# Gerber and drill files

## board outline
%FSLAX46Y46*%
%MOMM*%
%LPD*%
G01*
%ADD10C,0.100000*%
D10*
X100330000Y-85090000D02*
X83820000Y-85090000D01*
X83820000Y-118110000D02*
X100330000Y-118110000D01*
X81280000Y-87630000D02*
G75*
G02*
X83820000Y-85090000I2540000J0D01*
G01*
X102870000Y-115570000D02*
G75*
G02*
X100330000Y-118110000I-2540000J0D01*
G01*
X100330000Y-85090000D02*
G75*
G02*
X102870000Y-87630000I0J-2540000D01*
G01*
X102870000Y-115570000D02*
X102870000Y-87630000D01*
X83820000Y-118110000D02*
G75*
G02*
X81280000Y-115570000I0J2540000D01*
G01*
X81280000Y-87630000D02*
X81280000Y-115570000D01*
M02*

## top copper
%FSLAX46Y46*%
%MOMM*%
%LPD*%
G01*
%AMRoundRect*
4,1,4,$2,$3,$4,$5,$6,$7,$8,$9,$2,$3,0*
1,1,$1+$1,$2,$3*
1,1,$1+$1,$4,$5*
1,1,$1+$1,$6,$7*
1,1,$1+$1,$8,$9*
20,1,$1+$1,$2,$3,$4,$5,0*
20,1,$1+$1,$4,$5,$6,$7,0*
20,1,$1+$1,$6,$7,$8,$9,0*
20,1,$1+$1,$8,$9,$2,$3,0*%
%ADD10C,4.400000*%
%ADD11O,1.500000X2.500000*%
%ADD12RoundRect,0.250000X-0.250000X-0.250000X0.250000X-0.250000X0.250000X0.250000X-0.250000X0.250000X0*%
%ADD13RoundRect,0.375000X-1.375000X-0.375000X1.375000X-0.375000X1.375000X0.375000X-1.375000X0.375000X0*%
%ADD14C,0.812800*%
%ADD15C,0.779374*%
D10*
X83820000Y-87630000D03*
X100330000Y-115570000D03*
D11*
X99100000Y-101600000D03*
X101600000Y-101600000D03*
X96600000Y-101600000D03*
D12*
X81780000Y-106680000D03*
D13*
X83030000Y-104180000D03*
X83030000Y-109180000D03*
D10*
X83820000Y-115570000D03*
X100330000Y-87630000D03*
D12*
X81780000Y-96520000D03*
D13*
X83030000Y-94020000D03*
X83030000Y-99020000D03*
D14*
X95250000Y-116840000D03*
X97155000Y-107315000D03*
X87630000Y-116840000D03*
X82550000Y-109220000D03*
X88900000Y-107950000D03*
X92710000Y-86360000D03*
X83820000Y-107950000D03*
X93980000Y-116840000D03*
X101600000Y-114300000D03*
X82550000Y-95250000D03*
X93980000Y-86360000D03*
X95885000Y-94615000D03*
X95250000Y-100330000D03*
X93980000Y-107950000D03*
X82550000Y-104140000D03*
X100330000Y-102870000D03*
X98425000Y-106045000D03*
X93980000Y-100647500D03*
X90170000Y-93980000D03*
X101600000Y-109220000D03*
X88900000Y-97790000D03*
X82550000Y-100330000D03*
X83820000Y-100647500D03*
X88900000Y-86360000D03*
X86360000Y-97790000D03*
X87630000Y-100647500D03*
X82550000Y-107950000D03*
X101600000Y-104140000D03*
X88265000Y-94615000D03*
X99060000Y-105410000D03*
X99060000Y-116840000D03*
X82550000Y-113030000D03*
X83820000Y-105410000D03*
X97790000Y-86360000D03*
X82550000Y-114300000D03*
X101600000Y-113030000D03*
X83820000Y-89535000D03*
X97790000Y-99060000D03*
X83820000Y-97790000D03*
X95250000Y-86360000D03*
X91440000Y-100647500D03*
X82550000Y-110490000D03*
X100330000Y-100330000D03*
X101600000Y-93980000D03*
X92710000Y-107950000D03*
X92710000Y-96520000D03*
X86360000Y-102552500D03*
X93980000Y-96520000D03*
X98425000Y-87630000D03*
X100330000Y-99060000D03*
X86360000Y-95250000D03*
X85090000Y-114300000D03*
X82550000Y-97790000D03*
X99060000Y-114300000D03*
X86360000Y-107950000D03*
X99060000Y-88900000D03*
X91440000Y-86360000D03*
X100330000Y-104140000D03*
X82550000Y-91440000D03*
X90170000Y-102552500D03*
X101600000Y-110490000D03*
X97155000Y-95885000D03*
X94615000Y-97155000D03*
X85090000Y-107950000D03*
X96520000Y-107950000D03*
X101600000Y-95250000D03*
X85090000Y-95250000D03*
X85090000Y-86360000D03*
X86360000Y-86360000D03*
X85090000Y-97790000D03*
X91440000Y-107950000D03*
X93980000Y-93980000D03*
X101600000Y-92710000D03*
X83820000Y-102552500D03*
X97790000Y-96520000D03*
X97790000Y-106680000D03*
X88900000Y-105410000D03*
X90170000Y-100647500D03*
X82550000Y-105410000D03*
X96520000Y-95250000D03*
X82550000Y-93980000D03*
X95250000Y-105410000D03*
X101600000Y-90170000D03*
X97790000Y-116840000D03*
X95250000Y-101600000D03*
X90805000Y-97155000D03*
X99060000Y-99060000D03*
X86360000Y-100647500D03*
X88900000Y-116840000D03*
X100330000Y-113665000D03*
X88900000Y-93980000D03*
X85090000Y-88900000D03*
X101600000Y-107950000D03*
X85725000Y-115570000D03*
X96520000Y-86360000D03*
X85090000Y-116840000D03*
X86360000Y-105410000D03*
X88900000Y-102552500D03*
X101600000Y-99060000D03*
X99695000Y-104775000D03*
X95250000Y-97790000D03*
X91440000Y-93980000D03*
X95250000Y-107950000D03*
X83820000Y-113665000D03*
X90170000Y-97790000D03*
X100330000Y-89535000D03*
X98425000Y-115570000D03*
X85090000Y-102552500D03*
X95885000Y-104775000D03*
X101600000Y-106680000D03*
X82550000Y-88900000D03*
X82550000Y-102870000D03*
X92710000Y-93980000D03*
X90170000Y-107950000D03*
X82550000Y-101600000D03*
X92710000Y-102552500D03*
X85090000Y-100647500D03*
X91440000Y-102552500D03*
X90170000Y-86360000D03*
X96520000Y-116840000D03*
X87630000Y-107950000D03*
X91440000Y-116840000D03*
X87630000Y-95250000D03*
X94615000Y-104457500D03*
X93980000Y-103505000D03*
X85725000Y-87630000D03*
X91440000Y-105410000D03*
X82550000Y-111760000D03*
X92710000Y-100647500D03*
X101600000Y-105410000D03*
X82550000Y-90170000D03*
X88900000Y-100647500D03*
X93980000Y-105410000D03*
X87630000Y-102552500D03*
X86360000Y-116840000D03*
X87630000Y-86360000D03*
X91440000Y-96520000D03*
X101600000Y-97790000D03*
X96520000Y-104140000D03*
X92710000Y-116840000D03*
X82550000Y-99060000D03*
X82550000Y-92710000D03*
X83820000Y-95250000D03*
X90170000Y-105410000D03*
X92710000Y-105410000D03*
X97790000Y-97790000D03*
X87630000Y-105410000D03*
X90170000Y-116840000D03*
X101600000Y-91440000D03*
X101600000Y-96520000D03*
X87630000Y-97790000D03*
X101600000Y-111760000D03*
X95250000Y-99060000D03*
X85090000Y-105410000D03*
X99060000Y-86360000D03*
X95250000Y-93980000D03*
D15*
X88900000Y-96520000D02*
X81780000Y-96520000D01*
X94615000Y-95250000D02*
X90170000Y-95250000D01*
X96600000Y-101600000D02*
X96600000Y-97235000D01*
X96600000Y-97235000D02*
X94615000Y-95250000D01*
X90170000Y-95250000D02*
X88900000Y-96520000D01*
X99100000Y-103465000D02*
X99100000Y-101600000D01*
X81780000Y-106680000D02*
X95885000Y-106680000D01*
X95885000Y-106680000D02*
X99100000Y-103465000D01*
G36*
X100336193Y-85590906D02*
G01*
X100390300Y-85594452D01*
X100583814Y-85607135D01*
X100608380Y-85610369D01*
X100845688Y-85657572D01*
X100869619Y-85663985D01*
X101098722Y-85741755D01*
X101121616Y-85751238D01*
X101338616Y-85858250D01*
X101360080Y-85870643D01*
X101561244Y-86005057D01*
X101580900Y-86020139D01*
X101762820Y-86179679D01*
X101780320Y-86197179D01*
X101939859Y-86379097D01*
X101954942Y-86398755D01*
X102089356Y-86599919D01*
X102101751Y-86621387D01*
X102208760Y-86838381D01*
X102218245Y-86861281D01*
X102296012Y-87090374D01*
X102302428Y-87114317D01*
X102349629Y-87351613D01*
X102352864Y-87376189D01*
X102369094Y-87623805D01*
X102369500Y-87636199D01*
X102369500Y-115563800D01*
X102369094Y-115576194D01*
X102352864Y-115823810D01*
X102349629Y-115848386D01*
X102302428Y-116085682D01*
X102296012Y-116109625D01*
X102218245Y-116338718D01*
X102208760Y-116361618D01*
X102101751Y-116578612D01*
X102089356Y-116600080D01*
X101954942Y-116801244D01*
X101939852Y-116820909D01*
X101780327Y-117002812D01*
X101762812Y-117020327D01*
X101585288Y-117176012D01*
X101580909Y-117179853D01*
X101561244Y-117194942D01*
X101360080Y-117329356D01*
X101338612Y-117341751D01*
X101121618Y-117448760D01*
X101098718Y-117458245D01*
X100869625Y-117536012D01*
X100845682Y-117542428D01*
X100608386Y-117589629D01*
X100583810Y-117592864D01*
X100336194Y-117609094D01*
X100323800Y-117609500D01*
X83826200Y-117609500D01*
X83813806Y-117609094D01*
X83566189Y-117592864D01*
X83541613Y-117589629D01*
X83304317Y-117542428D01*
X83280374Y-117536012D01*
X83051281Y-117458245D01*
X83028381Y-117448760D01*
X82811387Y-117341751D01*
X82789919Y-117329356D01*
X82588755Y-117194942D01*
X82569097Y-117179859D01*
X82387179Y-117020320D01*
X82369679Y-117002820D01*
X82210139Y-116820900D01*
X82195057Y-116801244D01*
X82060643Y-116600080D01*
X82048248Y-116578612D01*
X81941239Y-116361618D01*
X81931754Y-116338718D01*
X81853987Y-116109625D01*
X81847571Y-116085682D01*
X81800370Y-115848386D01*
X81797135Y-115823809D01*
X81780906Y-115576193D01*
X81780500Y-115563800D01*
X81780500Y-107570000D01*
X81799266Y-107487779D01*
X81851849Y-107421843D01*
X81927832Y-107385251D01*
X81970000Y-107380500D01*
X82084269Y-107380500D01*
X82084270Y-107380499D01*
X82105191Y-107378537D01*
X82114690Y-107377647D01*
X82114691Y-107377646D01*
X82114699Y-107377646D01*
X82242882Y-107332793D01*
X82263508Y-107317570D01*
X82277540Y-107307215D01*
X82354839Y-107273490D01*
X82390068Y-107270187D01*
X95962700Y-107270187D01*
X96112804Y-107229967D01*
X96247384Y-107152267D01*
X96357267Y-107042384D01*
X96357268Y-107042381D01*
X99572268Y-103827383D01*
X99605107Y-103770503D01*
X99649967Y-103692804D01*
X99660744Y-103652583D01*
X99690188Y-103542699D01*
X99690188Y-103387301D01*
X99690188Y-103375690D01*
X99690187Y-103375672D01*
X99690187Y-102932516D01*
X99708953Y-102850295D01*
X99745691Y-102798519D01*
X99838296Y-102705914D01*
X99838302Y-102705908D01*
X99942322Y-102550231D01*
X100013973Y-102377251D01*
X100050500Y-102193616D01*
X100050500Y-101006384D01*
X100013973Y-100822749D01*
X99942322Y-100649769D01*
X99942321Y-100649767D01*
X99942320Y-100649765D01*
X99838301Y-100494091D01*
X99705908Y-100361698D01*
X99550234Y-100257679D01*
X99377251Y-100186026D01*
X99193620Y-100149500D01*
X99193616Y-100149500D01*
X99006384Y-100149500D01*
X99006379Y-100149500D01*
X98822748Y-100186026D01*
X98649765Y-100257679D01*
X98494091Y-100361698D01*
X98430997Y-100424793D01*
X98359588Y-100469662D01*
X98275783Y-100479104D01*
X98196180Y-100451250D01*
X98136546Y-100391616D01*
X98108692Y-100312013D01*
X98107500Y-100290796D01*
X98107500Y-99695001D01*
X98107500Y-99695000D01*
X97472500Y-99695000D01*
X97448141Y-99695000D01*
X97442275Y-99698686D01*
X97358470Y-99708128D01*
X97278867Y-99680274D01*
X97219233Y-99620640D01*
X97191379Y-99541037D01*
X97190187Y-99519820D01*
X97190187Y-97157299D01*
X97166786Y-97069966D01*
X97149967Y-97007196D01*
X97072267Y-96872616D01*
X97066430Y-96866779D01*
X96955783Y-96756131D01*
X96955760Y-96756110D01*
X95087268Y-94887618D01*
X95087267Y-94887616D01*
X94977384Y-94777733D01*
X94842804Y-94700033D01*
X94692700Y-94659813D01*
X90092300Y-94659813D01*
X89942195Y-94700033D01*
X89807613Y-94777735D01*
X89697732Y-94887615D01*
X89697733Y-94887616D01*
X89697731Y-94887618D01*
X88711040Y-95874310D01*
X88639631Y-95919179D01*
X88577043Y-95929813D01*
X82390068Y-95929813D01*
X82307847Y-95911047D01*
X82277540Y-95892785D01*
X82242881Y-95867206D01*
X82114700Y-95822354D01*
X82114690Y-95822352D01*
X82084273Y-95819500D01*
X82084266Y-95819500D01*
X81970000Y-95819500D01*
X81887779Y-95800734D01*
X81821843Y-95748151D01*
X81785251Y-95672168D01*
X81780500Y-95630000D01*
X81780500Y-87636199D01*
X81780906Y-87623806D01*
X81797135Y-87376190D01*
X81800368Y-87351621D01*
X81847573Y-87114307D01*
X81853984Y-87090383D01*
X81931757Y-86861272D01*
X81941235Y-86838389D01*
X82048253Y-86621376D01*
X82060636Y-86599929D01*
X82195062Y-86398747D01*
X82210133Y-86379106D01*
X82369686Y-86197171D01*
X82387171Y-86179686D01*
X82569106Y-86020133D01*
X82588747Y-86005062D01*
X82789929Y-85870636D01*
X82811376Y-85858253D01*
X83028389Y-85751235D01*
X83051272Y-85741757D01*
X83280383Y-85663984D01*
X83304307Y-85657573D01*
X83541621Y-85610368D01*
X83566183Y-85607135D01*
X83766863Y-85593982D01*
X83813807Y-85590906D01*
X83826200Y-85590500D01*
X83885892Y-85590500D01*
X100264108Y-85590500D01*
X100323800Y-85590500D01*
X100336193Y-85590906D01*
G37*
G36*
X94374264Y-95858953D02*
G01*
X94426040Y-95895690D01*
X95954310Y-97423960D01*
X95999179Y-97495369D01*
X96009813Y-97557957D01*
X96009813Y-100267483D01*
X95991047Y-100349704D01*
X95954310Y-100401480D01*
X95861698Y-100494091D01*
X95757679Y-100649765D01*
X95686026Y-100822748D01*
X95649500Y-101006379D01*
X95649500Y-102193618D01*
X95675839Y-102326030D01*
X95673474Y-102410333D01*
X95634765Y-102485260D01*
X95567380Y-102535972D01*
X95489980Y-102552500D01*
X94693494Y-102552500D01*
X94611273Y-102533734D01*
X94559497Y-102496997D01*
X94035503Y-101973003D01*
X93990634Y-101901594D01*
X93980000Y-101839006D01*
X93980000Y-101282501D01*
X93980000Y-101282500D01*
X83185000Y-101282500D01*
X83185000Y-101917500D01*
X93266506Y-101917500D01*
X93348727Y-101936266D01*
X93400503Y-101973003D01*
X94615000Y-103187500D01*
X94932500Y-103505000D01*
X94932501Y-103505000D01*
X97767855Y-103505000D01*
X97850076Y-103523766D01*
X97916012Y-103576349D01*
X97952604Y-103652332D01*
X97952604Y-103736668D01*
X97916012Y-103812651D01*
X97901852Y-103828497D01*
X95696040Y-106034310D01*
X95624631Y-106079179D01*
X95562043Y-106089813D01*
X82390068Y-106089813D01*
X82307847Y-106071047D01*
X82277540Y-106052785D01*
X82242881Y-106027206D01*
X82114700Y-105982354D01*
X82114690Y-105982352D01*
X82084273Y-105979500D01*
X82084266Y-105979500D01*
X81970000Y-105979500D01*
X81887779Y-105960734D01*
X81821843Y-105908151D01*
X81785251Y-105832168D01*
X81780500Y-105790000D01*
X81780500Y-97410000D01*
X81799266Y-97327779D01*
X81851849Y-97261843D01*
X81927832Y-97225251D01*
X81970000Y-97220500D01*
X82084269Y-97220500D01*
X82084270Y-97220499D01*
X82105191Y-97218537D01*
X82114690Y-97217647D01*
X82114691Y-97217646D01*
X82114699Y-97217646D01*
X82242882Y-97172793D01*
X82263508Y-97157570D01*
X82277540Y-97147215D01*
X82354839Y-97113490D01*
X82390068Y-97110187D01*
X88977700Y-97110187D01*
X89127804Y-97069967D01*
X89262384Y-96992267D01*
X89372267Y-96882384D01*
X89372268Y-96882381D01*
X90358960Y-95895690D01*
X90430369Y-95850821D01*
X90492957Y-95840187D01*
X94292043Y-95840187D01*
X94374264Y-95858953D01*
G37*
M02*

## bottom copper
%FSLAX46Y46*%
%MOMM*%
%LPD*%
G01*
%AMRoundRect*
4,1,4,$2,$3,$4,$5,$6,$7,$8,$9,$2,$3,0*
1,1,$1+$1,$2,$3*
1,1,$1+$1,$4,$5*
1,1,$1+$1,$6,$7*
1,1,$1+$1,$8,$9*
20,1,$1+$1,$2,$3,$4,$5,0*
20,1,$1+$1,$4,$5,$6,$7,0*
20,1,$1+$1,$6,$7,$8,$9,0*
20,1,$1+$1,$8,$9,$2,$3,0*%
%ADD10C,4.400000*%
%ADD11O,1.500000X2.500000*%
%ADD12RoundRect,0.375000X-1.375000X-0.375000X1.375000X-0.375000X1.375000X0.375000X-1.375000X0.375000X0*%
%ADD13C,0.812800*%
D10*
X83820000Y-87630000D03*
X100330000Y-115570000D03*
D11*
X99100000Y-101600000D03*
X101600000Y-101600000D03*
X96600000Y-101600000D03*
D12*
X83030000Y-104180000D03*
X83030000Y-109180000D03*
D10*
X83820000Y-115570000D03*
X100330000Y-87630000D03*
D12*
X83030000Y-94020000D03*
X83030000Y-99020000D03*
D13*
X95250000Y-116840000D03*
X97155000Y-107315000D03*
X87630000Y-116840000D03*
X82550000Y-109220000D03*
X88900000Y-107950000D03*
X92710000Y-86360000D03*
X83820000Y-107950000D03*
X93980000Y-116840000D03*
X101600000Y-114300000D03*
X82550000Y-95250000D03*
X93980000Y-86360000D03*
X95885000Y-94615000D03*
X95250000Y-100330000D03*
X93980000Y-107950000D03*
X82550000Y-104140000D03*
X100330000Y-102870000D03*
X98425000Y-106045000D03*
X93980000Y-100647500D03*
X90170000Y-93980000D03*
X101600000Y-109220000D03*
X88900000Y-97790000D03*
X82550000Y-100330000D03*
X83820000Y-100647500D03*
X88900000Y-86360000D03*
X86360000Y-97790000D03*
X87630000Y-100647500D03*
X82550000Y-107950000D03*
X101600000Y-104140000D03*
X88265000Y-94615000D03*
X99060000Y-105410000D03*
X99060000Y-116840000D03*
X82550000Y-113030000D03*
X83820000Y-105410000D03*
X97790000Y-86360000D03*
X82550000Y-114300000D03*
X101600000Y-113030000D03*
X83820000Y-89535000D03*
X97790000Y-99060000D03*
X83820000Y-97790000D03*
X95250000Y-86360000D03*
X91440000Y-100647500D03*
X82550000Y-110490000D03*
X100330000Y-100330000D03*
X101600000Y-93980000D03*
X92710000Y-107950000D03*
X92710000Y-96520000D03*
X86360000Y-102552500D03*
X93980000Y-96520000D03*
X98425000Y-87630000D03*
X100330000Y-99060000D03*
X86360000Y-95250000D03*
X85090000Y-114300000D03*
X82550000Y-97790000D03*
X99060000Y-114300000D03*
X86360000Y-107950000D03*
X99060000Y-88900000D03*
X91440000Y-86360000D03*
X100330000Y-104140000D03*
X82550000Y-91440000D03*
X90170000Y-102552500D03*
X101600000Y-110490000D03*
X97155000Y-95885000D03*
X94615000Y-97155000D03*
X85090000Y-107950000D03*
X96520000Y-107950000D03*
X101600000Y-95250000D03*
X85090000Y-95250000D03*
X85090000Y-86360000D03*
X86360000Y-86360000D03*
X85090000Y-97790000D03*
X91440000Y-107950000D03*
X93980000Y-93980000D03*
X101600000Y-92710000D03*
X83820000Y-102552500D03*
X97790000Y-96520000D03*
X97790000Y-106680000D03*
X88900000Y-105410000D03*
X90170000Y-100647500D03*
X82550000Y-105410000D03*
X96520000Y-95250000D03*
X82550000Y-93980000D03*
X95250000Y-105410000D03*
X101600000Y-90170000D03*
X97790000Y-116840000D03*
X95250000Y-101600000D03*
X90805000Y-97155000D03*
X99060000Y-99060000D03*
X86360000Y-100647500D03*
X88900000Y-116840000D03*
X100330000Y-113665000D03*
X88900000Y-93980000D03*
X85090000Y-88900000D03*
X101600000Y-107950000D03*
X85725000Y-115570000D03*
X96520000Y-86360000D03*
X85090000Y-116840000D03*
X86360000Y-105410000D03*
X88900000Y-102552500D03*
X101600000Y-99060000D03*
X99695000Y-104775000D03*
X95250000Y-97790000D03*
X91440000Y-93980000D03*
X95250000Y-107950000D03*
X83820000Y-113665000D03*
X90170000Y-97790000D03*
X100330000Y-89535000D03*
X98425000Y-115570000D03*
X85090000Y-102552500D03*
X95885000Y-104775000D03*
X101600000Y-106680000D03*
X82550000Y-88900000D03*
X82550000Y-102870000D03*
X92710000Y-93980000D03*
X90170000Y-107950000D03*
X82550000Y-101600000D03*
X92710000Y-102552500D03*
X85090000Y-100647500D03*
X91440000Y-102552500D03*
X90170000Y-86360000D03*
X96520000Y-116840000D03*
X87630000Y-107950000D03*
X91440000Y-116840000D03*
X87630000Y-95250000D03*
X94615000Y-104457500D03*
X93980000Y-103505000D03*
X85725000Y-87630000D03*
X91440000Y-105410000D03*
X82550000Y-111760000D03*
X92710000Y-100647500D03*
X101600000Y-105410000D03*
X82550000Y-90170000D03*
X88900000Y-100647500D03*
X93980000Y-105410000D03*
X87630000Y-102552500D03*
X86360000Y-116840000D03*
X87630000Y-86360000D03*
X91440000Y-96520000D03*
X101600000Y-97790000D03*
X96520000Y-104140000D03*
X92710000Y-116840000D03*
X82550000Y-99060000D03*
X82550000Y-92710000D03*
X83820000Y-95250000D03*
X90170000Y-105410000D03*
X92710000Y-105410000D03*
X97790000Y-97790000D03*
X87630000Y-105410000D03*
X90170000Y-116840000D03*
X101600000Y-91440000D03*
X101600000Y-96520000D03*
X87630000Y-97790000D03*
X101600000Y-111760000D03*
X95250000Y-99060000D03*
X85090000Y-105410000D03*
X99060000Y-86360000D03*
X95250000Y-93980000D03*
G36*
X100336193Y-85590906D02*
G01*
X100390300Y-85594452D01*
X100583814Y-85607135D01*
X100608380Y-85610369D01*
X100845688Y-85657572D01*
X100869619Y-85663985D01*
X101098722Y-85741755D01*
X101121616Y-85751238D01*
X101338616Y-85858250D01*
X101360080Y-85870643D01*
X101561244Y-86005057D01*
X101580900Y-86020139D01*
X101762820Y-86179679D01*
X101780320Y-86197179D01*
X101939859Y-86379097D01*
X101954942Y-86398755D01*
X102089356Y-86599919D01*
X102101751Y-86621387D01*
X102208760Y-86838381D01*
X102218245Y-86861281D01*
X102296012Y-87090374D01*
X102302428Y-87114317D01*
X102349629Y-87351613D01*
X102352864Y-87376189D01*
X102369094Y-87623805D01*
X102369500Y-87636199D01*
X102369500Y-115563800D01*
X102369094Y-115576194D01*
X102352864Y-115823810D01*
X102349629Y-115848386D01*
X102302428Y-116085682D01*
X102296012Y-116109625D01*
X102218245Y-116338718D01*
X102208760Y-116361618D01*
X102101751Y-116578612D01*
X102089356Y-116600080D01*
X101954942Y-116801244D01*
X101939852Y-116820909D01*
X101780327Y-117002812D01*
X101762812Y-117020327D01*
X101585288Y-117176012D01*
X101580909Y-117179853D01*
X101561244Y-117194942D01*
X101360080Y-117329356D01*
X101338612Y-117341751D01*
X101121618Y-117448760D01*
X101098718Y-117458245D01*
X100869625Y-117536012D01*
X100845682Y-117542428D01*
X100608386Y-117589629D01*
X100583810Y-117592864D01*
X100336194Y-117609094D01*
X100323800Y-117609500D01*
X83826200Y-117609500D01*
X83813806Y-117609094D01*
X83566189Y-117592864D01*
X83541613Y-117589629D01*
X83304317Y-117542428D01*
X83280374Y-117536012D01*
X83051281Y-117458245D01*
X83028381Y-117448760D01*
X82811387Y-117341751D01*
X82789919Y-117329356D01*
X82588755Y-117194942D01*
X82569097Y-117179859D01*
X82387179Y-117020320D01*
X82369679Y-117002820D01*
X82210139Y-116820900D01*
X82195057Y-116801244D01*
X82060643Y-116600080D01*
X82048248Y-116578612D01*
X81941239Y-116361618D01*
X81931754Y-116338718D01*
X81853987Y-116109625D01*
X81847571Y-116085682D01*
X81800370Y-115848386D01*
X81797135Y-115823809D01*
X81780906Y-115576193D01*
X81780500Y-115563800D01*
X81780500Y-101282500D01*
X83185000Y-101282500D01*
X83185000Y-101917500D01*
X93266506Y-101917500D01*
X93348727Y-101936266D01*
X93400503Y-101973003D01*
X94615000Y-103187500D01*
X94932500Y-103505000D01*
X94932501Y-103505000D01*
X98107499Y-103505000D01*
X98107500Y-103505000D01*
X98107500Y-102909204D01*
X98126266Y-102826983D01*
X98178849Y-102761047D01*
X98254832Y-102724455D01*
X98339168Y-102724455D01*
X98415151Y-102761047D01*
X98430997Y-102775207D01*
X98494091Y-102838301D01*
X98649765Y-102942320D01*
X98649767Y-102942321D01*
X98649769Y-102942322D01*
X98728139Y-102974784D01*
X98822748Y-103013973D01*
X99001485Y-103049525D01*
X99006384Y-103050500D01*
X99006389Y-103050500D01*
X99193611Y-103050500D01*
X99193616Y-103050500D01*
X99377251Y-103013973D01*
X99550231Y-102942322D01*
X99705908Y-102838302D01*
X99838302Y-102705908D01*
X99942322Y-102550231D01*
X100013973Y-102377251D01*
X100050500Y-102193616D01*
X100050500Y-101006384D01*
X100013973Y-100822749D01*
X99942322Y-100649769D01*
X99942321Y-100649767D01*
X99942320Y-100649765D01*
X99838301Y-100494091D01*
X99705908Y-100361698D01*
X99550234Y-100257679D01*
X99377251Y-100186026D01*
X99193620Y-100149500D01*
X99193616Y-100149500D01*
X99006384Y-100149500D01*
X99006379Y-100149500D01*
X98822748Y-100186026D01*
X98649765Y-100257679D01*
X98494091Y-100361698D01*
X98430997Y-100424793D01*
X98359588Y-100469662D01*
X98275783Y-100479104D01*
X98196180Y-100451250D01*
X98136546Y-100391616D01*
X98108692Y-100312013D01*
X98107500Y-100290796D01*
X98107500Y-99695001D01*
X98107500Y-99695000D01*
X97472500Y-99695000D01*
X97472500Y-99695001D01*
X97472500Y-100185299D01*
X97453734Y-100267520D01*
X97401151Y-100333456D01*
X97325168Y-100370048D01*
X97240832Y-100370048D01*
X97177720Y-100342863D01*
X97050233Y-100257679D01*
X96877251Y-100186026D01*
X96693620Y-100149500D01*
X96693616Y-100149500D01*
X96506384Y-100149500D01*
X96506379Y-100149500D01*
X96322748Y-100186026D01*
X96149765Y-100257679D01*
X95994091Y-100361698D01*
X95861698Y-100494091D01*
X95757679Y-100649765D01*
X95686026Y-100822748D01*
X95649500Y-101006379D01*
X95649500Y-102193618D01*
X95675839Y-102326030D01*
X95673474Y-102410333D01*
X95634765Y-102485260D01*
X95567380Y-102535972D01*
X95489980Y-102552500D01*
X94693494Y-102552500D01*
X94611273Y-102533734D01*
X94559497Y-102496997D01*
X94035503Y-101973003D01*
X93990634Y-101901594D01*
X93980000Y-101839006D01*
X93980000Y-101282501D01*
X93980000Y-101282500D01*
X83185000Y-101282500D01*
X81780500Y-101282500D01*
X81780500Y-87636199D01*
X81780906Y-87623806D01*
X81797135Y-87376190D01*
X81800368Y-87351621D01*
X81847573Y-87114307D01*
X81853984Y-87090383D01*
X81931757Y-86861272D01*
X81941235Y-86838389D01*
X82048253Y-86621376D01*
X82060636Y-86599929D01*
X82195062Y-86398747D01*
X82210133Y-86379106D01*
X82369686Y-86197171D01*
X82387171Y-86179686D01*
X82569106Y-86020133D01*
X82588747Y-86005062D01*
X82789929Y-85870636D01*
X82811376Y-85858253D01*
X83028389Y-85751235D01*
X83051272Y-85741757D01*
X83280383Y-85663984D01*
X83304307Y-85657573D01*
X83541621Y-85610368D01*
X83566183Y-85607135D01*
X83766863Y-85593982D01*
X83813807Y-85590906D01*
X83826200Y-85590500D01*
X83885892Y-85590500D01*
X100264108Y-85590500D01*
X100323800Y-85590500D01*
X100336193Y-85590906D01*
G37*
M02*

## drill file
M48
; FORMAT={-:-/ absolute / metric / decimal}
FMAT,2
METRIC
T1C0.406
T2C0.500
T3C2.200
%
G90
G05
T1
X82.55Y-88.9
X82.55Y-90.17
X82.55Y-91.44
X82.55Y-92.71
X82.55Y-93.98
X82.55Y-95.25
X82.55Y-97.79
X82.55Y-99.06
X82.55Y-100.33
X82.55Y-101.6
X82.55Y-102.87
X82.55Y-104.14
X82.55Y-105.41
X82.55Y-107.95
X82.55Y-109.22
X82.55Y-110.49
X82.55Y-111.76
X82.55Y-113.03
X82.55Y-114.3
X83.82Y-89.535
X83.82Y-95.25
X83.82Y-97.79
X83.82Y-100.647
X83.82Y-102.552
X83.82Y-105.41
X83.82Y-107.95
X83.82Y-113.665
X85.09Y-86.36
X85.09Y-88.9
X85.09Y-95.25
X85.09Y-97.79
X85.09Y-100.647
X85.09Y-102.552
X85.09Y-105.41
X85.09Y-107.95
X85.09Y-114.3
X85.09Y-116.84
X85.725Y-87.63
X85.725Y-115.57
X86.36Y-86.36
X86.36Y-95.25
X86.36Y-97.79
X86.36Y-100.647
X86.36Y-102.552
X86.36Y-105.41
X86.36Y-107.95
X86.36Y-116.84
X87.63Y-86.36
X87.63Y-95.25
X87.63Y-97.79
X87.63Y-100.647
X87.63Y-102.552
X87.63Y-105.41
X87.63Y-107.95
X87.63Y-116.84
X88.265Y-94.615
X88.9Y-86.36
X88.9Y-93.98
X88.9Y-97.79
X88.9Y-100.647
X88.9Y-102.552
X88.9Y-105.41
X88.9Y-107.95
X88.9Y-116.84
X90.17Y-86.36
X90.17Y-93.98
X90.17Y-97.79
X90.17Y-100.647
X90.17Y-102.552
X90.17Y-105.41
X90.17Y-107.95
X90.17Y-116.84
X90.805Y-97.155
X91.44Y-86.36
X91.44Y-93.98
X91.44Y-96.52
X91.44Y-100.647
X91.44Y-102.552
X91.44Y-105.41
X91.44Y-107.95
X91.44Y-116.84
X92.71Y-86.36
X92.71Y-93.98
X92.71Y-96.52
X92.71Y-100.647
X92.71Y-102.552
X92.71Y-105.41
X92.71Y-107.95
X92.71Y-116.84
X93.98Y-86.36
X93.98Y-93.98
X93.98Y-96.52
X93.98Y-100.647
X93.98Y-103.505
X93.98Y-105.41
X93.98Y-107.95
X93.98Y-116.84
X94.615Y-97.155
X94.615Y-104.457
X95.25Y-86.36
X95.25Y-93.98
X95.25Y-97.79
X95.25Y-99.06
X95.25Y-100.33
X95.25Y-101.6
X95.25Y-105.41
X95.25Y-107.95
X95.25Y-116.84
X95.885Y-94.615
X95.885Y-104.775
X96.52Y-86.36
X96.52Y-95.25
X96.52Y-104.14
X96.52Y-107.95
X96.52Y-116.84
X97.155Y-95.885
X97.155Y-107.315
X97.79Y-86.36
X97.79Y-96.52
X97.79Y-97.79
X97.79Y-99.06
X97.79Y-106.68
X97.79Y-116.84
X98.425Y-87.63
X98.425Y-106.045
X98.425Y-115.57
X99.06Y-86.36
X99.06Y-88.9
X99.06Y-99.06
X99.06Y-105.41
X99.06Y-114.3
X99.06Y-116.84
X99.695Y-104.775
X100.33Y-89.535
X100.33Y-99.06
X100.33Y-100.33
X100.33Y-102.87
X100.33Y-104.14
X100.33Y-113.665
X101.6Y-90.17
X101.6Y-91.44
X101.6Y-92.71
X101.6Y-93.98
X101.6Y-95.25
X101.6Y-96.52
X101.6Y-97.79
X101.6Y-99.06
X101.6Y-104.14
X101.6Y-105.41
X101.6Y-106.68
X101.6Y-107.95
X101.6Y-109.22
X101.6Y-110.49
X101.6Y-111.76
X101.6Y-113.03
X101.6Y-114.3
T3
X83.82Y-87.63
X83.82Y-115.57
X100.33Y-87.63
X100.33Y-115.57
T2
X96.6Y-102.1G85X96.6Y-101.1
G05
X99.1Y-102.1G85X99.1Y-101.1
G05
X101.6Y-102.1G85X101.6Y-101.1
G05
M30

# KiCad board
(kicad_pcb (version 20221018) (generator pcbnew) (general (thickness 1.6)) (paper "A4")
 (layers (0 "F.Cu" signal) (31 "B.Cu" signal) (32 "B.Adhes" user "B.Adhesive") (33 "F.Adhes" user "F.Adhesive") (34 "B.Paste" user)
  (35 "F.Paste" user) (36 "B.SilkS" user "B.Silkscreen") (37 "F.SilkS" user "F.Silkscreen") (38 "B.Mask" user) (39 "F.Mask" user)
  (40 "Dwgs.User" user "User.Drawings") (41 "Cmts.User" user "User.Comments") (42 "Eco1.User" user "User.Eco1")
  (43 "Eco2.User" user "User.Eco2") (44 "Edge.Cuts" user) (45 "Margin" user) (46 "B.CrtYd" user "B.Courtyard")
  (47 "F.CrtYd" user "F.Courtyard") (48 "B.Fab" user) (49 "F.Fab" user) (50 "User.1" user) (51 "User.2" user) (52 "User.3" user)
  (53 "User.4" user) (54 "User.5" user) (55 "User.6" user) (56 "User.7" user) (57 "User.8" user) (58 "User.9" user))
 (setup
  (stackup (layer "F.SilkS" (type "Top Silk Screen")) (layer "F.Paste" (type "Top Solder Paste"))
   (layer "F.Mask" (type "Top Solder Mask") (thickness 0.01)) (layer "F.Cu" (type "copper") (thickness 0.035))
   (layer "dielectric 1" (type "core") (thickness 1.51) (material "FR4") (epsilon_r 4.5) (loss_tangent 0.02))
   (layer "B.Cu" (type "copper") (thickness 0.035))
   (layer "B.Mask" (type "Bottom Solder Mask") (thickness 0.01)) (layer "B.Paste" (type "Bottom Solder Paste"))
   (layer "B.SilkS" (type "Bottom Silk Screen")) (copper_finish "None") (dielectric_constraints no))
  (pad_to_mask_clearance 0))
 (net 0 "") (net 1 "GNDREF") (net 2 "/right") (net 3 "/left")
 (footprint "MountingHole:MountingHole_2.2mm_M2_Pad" (layer "F.Cu") (at 83.82 87.63)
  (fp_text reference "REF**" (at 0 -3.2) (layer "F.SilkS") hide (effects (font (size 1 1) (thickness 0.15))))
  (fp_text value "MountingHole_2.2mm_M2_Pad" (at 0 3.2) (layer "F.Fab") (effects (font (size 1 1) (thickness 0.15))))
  (pad "1" thru_hole circle (at 0 0) (size 4.4 4.4) (drill 2.2) (layers "*.Cu" "*.Mask") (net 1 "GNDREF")))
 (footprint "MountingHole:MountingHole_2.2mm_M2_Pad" (layer "F.Cu") (at 100.33 115.57)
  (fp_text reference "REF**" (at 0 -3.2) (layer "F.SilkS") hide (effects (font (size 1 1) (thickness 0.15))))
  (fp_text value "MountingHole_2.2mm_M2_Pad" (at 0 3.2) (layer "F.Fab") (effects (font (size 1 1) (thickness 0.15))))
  (pad "1" thru_hole circle (at 0 0) (size 4.4 4.4) (drill 2.2) (layers "*.Cu" "*.Mask") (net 1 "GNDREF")))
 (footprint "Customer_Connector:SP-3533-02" (layer "F.Cu") (at 101.6 101.6 180)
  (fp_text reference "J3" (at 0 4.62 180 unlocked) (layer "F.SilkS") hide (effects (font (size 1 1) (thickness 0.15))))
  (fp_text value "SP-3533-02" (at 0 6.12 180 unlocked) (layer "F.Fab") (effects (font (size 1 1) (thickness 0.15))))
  (pad "R" thru_hole oval (at 2.5 0 180) (size 1.5 2.5) (drill oval 0.5 1.5) (layers "*.Cu" "*.Mask") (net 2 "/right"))
  (pad "S" thru_hole oval (at 0 0 180) (size 1.5 2.5) (drill oval 0.5 1.5) (layers "*.Cu" "*.Mask") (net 1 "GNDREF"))
  (pad "T" thru_hole oval (at 5 0 180) (size 1.5 2.5) (drill oval 0.5 1.5) (layers "*.Cu" "*.Mask") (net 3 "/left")))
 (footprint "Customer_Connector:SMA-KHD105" (layer "F.Cu") (at 81.28 106.68)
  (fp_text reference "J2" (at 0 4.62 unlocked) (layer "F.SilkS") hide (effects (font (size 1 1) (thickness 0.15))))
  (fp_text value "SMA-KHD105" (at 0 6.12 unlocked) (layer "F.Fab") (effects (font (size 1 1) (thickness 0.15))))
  (pad "1" smd roundrect (at 0.5 0) (size 1 1) (layers "F.Cu" "F.Paste" "F.Mask") (roundrect_rratio 0.25) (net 2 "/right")
   (thermal_bridge_angle 45))
  (pad "2" smd roundrect (at 1.75 -2.5) (size 3.5 1.5) (layers "F.Cu" "F.Paste" "F.Mask") (roundrect_rratio 0.25) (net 1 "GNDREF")
   (thermal_bridge_angle 45))
  (pad "2" smd roundrect (at 1.75 -2.5) (size 3.5 1.5) (layers "B.Cu" "B.Paste" "B.Mask") (roundrect_rratio 0.25) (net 1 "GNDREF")
   (thermal_bridge_angle 45))
  (pad "2" smd roundrect (at 1.75 2.5) (size 3.5 1.5) (layers "F.Cu" "F.Paste" "F.Mask") (roundrect_rratio 0.25) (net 1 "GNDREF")
   (thermal_bridge_angle 45))
  (pad "2" smd roundrect (at 1.75 2.5) (size 3.5 1.5) (layers "B.Cu" "B.Paste" "B.Mask") (roundrect_rratio 0.25) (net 1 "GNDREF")
   (thermal_bridge_angle 45)))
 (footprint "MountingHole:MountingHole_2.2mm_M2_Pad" (layer "F.Cu") (at 83.82 115.57)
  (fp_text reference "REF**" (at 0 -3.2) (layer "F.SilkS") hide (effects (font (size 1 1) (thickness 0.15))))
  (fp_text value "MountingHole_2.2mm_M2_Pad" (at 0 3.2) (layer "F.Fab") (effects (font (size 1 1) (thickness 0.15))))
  (pad "1" thru_hole circle (at 0 0) (size 4.4 4.4) (drill 2.2) (layers "*.Cu" "*.Mask") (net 1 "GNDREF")))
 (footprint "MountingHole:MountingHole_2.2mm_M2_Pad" (layer "F.Cu") (at 100.33 87.63)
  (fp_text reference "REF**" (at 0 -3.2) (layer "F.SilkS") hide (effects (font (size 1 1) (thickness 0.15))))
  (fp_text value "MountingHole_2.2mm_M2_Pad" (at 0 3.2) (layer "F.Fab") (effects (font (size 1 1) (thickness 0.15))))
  (pad "1" thru_hole circle (at 0 0) (size 4.4 4.4) (drill 2.2) (layers "*.Cu" "*.Mask") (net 1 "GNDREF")))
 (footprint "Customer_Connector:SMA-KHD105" (layer "F.Cu") (at 81.28 96.52)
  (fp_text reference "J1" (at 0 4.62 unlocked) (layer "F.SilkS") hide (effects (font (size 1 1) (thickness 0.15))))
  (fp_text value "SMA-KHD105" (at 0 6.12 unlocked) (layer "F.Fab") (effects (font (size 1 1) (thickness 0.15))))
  (pad "1" smd roundrect (at 0.5 0) (size 1 1) (layers "F.Cu" "F.Paste" "F.Mask") (roundrect_rratio 0.25) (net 3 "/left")
   (thermal_bridge_angle 45))
  (pad "2" smd roundrect (at 1.75 -2.5) (size 3.5 1.5) (layers "F.Cu" "F.Paste" "F.Mask") (roundrect_rratio 0.25) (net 1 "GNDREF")
   (thermal_bridge_angle 45))
  (pad "2" smd roundrect (at 1.75 -2.5) (size 3.5 1.5) (layers "B.Cu" "B.Paste" "B.Mask") (roundrect_rratio 0.25) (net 1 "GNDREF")
   (thermal_bridge_angle 45))
  (pad "2" smd roundrect (at 1.75 2.5) (size 3.5 1.5) (layers "F.Cu" "F.Paste" "F.Mask") (roundrect_rratio 0.25) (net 1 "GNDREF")
   (thermal_bridge_angle 45))
  (pad "2" smd roundrect (at 1.75 2.5) (size 3.5 1.5) (layers "B.Cu" "B.Paste" "B.Mask") (roundrect_rratio 0.25) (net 1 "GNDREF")
   (thermal_bridge_angle 45)))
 (gr_line (start 100.33 85.09) (end 83.82 85.09) (stroke (width 0.1) (type default)) (layer "Edge.Cuts"))
 (gr_line (start 83.82 118.11) (end 100.33 118.11) (stroke (width 0.1) (type default)) (layer "Edge.Cuts"))
 (gr_arc (start 81.28 87.63) (mid 82.023949 85.833949) (end 83.82 85.09) (stroke (width 0.1) (type default)) (layer "Edge.Cuts"))
 (gr_arc (start 102.87 115.57) (mid 102.126051 117.366051) (end 100.33 118.11) (stroke (width 0.1) (type default)) (layer "Edge.Cuts"))
 (gr_arc (start 100.33 85.09) (mid 102.126051 85.833949) (end 102.87 87.63) (stroke (width 0.1) (type default)) (layer "Edge.Cuts"))
 (gr_line (start 102.87 115.57) (end 102.87 87.63) (stroke (width 0.1) (type default)) (layer "Edge.Cuts"))
 (gr_arc (start 83.82 118.11) (mid 82.023949 117.366051) (end 81.28 115.57) (stroke (width 0.1) (type default)) (layer "Edge.Cuts"))
 (gr_line (start 81.28 87.63) (end 81.28 115.57) (stroke (width 0.1) (type default)) (layer "Edge.Cuts"))
 (segment (start 88.9 96.52) (end 81.78 96.52) (width 0.779374) (layer "F.Cu") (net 3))
 (segment (start 94.615 95.25) (end 90.17 95.25) (width 0.779374) (layer "F.Cu") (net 3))
 (segment (start 96.6 101.6) (end 96.6 97.235) (width 0.779374) (layer "F.Cu") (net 3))
 (segment (start 96.6 97.235) (end 94.615 95.25) (width 0.779374) (layer "F.Cu") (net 3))
 (segment (start 90.17 95.25) (end 88.9 96.52) (width 0.779374) (layer "F.Cu") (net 3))
 (via (at 95.25 116.84) (size 0.8128) (drill 0.4064) (layers "F.Cu" "B.Cu") (free) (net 1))
 (via (at 97.155 107.315) (size 0.8128) (drill 0.4064) (layers "F.Cu" "B.Cu") (free) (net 1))
 (via (at 87.63 116.84) (size 0.8128) (drill 0.4064) (layers "F.Cu" "B.Cu") (free) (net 1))
 (via (at 82.55 109.22) (size 0.8128) (drill 0.4064) (layers "F.Cu" "B.Cu") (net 1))
 (via (at 88.9 107.95) (size 0.8128) (drill 0.4064) (layers "F.Cu" "B.Cu") (free) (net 1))
 (via (at 92.71 86.36) (size 0.8128) (drill 0.4064) (layers "F.Cu" "B.Cu") (free) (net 1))
 (via (at 83.82 107.95) (size 0.8128) (drill 0.4064) (layers "F.Cu" "B.Cu") (free) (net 1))
 (via (at 93.98 116.84) (size 0.8128) (drill 0.4064) (layers "F.Cu" "B.Cu") (free) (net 1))
 (via (at 101.6 114.3) (size 0.8128) (drill 0.4064) (layers "F.Cu" "B.Cu") (free) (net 1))
 (via (at 82.55 95.25) (size 0.8128) (drill 0.4064) (layers "F.Cu" "B.Cu") (free) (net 1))
 (via (at 93.98 86.36) (size 0.8128) (drill 0.4064) (layers "F.Cu" "B.Cu") (free) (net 1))
 (via (at 95.885 94.615) (size 0.8128) (drill 0.4064) (layers "F.Cu" "B.Cu") (free) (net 1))
 (via (at 95.25 100.33) (size 0.8128) (drill 0.4064) (layers "F.Cu" "B.Cu") (free) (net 1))
 (via (at 93.98 107.95) (size 0.8128) (drill 0.4064) (layers "F.Cu" "B.Cu") (free) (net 1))
 (via (at 82.55 104.14) (size 0.8128) (drill 0.4064) (layers "F.Cu" "B.Cu") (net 1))
 (via (at 100.33 102.87) (size 0.8128) (drill 0.4064) (layers "F.Cu" "B.Cu") (free) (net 1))
 (via (at 98.425 106.045) (size 0.8128) (drill 0.4064) (layers "F.Cu" "B.Cu") (free) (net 1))
 (via (at 93.98 100.6475) (size 0.8128) (drill 0.4064) (layers "F.Cu" "B.Cu") (free) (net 1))
 (via (at 90.17 93.98) (size 0.8128) (drill 0.4064) (layers "F.Cu" "B.Cu") (free) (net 1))
 (via (at 101.6 109.22) (size 0.8128) (drill 0.4064) (layers "F.Cu" "B.Cu") (free) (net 1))
 (via (at 88.9 97.79) (size 0.8128) (drill 0.4064) (layers "F.Cu" "B.Cu") (free) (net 1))
 (via (at 82.55 100.33) (size 0.8128) (drill 0.4064) (layers "F.Cu" "B.Cu") (free) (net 1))
 (via (at 83.82 100.6475) (size 0.8128) (drill 0.4064) (layers "F.Cu" "B.Cu") (free) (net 1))
 (via (at 88.9 86.36) (size 0.8128) (drill 0.4064) (layers "F.Cu" "B.Cu") (free) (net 1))
 (via (at 86.36 97.79) (size 0.8128) (drill 0.4064) (layers "F.Cu" "B.Cu") (free) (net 1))
 (via (at 87.63 100.6475) (size 0.8128) (drill 0.4064) (layers "F.Cu" "B.Cu") (free) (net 1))
 (via (at 82.55 107.95) (size 0.8128) (drill 0.4064) (layers "F.Cu" "B.Cu") (free) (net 1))
 (via (at 101.6 104.14) (size 0.8128) (drill 0.4064) (layers "F.Cu" "B.Cu") (free) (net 1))
 (via (at 88.265 94.615) (size 0.8128) (drill 0.4064) (layers "F.Cu" "B.Cu") (free) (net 1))
 (via (at 99.06 105.41) (size 0.8128) (drill 0.4064) (layers "F.Cu" "B.Cu") (free) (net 1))
 (via (at 99.06 116.84) (size 0.8128) (drill 0.4064) (layers "F.Cu" "B.Cu") (free) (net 1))
 (via (at 82.55 113.03) (size 0.8128) (drill 0.4064) (layers "F.Cu" "B.Cu") (free) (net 1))
 (via (at 83.82 105.41) (size 0.8128) (drill 0.4064) (layers "F.Cu" "B.Cu") (free) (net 1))
 (via (at 97.79 86.36) (size 0.8128) (drill 0.4064) (layers "F.Cu" "B.Cu") (free) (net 1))
 (via (at 82.55 114.3) (size 0.8128) (drill 0.4064) (layers "F.Cu" "B.Cu") (free) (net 1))
 (via (at 101.6 113.03) (size 0.8128) (drill 0.4064) (layers "F.Cu" "B.Cu") (free) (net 1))
 (via (at 83.82 89.535) (size 0.8128) (drill 0.4064) (layers "F.Cu" "B.Cu") (free) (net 1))
 (via (at 97.79 99.06) (size 0.8128) (drill 0.4064) (layers "F.Cu" "B.Cu") (free) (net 1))
 (via (at 83.82 97.79) (size 0.8128) (drill 0.4064) (layers "F.Cu" "B.Cu") (free) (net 1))
 (via (at 95.25 86.36) (size 0.8128) (drill 0.4064) (layers "F.Cu" "B.Cu") (free) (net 1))
 (via (at 91.44 100.6475) (size 0.8128) (drill 0.4064) (layers "F.Cu" "B.Cu") (free) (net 1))
 (via (at 82.55 110.49) (size 0.8128) (drill 0.4064) (layers "F.Cu" "B.Cu") (free) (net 1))
 (via (at 100.33 100.33) (size 0.8128) (drill 0.4064) (layers "F.Cu" "B.Cu") (free) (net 1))
 (via (at 101.6 93.98) (size 0.8128) (drill 0.4064) (layers "F.Cu" "B.Cu") (free) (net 1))
 (via (at 92.71 107.95) (size 0.8128) (drill 0.4064) (layers "F.Cu" "B.Cu") (free) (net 1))
 (via (at 92.71 96.52) (size 0.8128) (drill 0.4064) (layers "F.Cu" "B.Cu") (free) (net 1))
 (via (at 86.36 102.5525) (size 0.8128) (drill 0.4064) (layers "F.Cu" "B.Cu") (free) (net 1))
 (via (at 93.98 96.52) (size 0.8128) (drill 0.4064) (layers "F.Cu" "B.Cu") (free) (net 1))
 (via (at 98.425 87.63) (size 0.8128) (drill 0.4064) (layers "F.Cu" "B.Cu") (free) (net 1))
 (via (at 100.33 99.06) (size 0.8128) (drill 0.4064) (layers "F.Cu" "B.Cu") (free) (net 1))
 (via (at 86.36 95.25) (size 0.8128) (drill 0.4064) (layers "F.Cu" "B.Cu") (free) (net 1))
 (via (at 85.09 114.3) (size 0.8128) (drill 0.4064) (layers "F.Cu" "B.Cu") (free) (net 1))
 (via (at 82.55 97.79) (size 0.8128) (drill 0.4064) (layers "F.Cu" "B.Cu") (free) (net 1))
 (via (at 99.06 114.3) (size 0.8128) (drill 0.4064) (layers "F.Cu" "B.Cu") (free) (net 1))
 (via (at 86.36 107.95) (size 0.8128) (drill 0.4064) (layers "F.Cu" "B.Cu") (free) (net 1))
 (via (at 99.06 88.9) (size 0.8128) (drill 0.4064) (layers "F.Cu" "B.Cu") (free) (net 1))
 (via (at 91.44 86.36) (size 0.8128) (drill 0.4064) (layers "F.Cu" "B.Cu") (free) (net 1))
 (via (at 100.33 104.14) (size 0.8128) (drill 0.4064) (layers "F.Cu" "B.Cu") (free) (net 1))
 (via (at 82.55 91.44) (size 0.8128) (drill 0.4064) (layers "F.Cu" "B.Cu") (free) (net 1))
 (via (at 90.17 102.5525) (size 0.8128) (drill 0.4064) (layers "F.Cu" "B.Cu") (free) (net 1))
 (via (at 101.6 110.49) (size 0.8128) (drill 0.4064) (layers "F.Cu" "B.Cu") (free) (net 1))
 (via (at 97.155 95.885) (size 0.8128) (drill 0.4064) (layers "F.Cu" "B.Cu") (free) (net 1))
 (via (at 94.615 97.155) (size 0.8128) (drill 0.4064) (layers "F.Cu" "B.Cu") (free) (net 1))
 (via (at 85.09 107.95) (size 0.8128) (drill 0.4064) (layers "F.Cu" "B.Cu") (free) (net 1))
 (via (at 96.52 107.95) (size 0.8128) (drill 0.4064) (layers "F.Cu" "B.Cu") (free) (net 1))
 (via (at 101.6 95.25) (size 0.8128) (drill 0.4064) (layers "F.Cu" "B.Cu") (free) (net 1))
 (via (at 85.09 95.25) (size 0.8128) (drill 0.4064) (layers "F.Cu" "B.Cu") (free) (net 1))
 (via (at 85.09 86.36) (size 0.8128) (drill 0.4064) (layers "F.Cu" "B.Cu") (free) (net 1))
 (via (at 86.36 86.36) (size 0.8128) (drill 0.4064) (layers "F.Cu" "B.Cu") (free) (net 1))
 (via (at 85.09 97.79) (size 0.8128) (drill 0.4064) (layers "F.Cu" "B.Cu") (free) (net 1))
 (via (at 91.44 107.95) (size 0.8128) (drill 0.4064) (layers "F.Cu" "B.Cu") (free) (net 1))
 (via (at 93.98 93.98) (size 0.8128) (drill 0.4064) (layers "F.Cu" "B.Cu") (free) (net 1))
 (via (at 101.6 92.71) (size 0.8128) (drill 0.4064) (layers "F.Cu" "B.Cu") (free) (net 1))
 (via (at 83.82 102.5525) (size 0.8128) (drill 0.4064) (layers "F.Cu" "B.Cu") (free) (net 1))
 (via (at 97.79 96.52) (size 0.8128) (drill 0.4064) (layers "F.Cu" "B.Cu") (free) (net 1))
 (via (at 97.79 106.68) (size 0.8128) (drill 0.4064) (layers "F.Cu" "B.Cu") (free) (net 1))
 (via (at 88.9 105.41) (size 0.8128) (drill 0.4064) (layers "F.Cu" "B.Cu") (free) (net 1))
 (via (at 90.17 100.6475) (size 0.8128) (drill 0.4064) (layers "F.Cu" "B.Cu") (free) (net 1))
 (via (at 82.55 105.41) (size 0.8128) (drill 0.4064) (layers "F.Cu" "B.Cu") (free) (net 1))
 (via (at 96.52 95.25) (size 0.8128) (drill 0.4064) (layers "F.Cu" "B.Cu") (free) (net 1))
 (via (at 82.55 93.98) (size 0.8128) (drill 0.4064) (layers "F.Cu" "B.Cu") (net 1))
 (via (at 95.25 105.41) (size 0.8128) (drill 0.4064) (layers "F.Cu" "B.Cu") (free) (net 1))
 (via (at 101.6 90.17) (size 0.8128) (drill 0.4064) (layers "F.Cu" "B.Cu") (free) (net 1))
 (via (at 97.79 116.84) (size 0.8128) (drill 0.4064) (layers "F.Cu" "B.Cu") (free) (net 1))
 (via (at 95.25 101.6) (size 0.8128) (drill 0.4064) (layers "F.Cu" "B.Cu") (free) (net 1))
 (via (at 90.805 97.155) (size 0.8128) (drill 0.4064) (layers "F.Cu" "B.Cu") (free) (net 1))
 (via (at 99.06 99.06) (size 0.8128) (drill 0.4064) (layers "F.Cu" "B.Cu") (free) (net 1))
 (via (at 86.36 100.6475) (size 0.8128) (drill 0.4064) (layers "F.Cu" "B.Cu") (free) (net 1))
 (via (at 88.9 116.84) (size 0.8128) (drill 0.4064) (layers "F.Cu" "B.Cu") (free) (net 1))
 (via (at 100.33 113.665) (size 0.8128) (drill 0.4064) (layers "F.Cu" "B.Cu") (free) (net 1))
 (via (at 88.9 93.98) (size 0.8128) (drill 0.4064) (layers "F.Cu" "B.Cu") (free) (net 1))
 (via (at 85.09 88.9) (size 0.8128) (drill 0.4064) (layers "F.Cu" "B.Cu") (free) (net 1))
 (via (at 101.6 107.95) (size 0.8128) (drill 0.4064) (layers "F.Cu" "B.Cu") (free) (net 1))
 (via (at 85.725 115.57) (size 0.8128) (drill 0.4064) (layers "F.Cu" "B.Cu") (free) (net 1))
 (via (at 96.52 86.36) (size 0.8128) (drill 0.4064) (layers "F.Cu" "B.Cu") (free) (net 1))
 (via (at 85.09 116.84) (size 0.8128) (drill 0.4064) (layers "F.Cu" "B.Cu") (free) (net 1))
 (via (at 86.36 105.41) (size 0.8128) (drill 0.4064) (layers "F.Cu" "B.Cu") (free) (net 1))
 (via (at 88.9 102.5525) (size 0.8128) (drill 0.4064) (layers "F.Cu" "B.Cu") (free) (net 1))
 (via (at 101.6 99.06) (size 0.8128) (drill 0.4064) (layers "F.Cu" "B.Cu") (free) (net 1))
 (via (at 99.695 104.775) (size 0.8128) (drill 0.4064) (layers "F.Cu" "B.Cu") (free) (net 1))
 (via (at 95.25 97.79) (size 0.8128) (drill 0.4064) (layers "F.Cu" "B.Cu") (free) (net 1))
 (via (at 91.44 93.98) (size 0.8128) (drill 0.4064) (layers "F.Cu" "B.Cu") (free) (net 1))
 (via (at 95.25 107.95) (size 0.8128) (drill 0.4064) (layers "F.Cu" "B.Cu") (free) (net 1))
 (via (at 83.82 113.665) (size 0.8128) (drill 0.4064) (layers "F.Cu" "B.Cu") (free) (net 1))
 (via (at 90.17 97.79) (size 0.8128) (drill 0.4064) (layers "F.Cu" "B.Cu") (free) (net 1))
 (via (at 100.33 89.535) (size 0.8128) (drill 0.4064) (layers "F.Cu" "B.Cu") (free) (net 1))
 (via (at 98.425 115.57) (size 0.8128) (drill 0.4064) (layers "F.Cu" "B.Cu") (free) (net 1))
 (via (at 85.09 102.5525) (size 0.8128) (drill 0.4064) (layers "F.Cu" "B.Cu") (free) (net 1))
 (via (at 95.885 104.775) (size 0.8128) (drill 0.4064) (layers "F.Cu" "B.Cu") (free) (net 1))
 (via (at 101.6 106.68) (size 0.8128) (drill 0.4064) (layers "F.Cu" "B.Cu") (free) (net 1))
 (via (at 82.55 88.9) (size 0.8128) (drill 0.4064) (layers "F.Cu" "B.Cu") (free) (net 1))
 (via (at 82.55 102.87) (size 0.8128) (drill 0.4064) (layers "F.Cu" "B.Cu") (free) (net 1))
 (via (at 92.71 93.98) (size 0.8128) (drill 0.4064) (layers "F.Cu" "B.Cu") (free) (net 1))
 (via (at 90.17 107.95) (size 0.8128) (drill 0.4064) (layers "F.Cu" "B.Cu") (free) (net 1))
 (via (at 82.55 101.6) (size 0.8128) (drill 0.4064) (layers "F.Cu" "B.Cu") (free) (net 1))
 (via (at 92.71 102.5525) (size 0.8128) (drill 0.4064) (layers "F.Cu" "B.Cu") (free) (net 1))
 (via (at 85.09 100.6475) (size 0.8128) (drill 0.4064) (layers "F.Cu" "B.Cu") (free) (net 1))
 (via (at 91.44 102.5525) (size 0.8128) (drill 0.4064) (layers "F.Cu" "B.Cu") (free) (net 1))
 (via (at 90.17 86.36) (size 0.8128) (drill 0.4064) (layers "F.Cu" "B.Cu") (free) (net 1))
 (via (at 96.52 116.84) (size 0.8128) (drill 0.4064) (layers "F.Cu" "B.Cu") (free) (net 1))
 (via (at 87.63 107.95) (size 0.8128) (drill 0.4064) (layers "F.Cu" "B.Cu") (free) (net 1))
 (via (at 91.44 116.84) (size 0.8128) (drill 0.4064) (layers "F.Cu" "B.Cu") (free) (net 1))
 (via (at 87.63 95.25) (size 0.8128) (drill 0.4064) (layers "F.Cu" "B.Cu") (free) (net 1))
 (via (at 94.615 104.4575) (size 0.8128) (drill 0.4064) (layers "F.Cu" "B.Cu") (free) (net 1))
 (via (at 93.98 103.505) (size 0.8128) (drill 0.4064) (layers "F.Cu" "B.Cu") (free) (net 1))
 (via (at 85.725 87.63) (size 0.8128) (drill 0.4064) (layers "F.Cu" "B.Cu") (free) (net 1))
 (via (at 91.44 105.41) (size 0.8128) (drill 0.4064) (layers "F.Cu" "B.Cu") (free) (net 1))
 (via (at 82.55 111.76) (size 0.8128) (drill 0.4064) (layers "F.Cu" "B.Cu") (free) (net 1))
 (via (at 92.71 100.6475) (size 0.8128) (drill 0.4064) (layers "F.Cu" "B.Cu") (free) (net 1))
 (via (at 101.6 105.41) (size 0.8128) (drill 0.4064) (layers "F.Cu" "B.Cu") (free) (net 1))
 (via (at 82.55 90.17) (size 0.8128) (drill 0.4064) (layers "F.Cu" "B.Cu") (free) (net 1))
 (via (at 88.9 100.6475) (size 0.8128) (drill 0.4064) (layers "F.Cu" "B.Cu") (free) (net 1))
 (via (at 93.98 105.41) (size 0.8128) (drill 0.4064) (layers "F.Cu" "B.Cu") (free) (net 1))
 (via (at 87.63 102.5525) (size 0.8128) (drill 0.4064) (layers "F.Cu" "B.Cu") (free) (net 1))
 (via (at 86.36 116.84) (size 0.8128) (drill 0.4064) (layers "F.Cu" "B.Cu") (free) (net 1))
 (via (at 87.63 86.36) (size 0.8128) (drill 0.4064) (layers "F.Cu" "B.Cu") (free) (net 1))
 (via (at 91.44 96.52) (size 0.8128) (drill 0.4064) (layers "F.Cu" "B.Cu") (free) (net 1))
 (via (at 101.6 97.79) (size 0.8128) (drill 0.4064) (layers "F.Cu" "B.Cu") (free) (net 1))
 (via (at 96.52 104.14) (size 0.8128) (drill 0.4064) (layers "F.Cu" "B.Cu") (free) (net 1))
 (via (at 92.71 116.84) (size 0.8128) (drill 0.4064) (layers "F.Cu" "B.Cu") (free) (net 1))
 (via (at 82.55 99.06) (size 0.8128) (drill 0.4064) (layers "F.Cu" "B.Cu") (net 1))
 (via (at 82.55 92.71) (size 0.8128) (drill 0.4064) (layers "F.Cu" "B.Cu") (free) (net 1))
 (via (at 83.82 95.25) (size 0.8128) (drill 0.4064) (layers "F.Cu" "B.Cu") (free) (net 1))
 (via (at 90.17 105.41) (size 0.8128) (drill 0.4064) (layers "F.Cu" "B.Cu") (free) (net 1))
 (via (at 92.71 105.41) (size 0.8128) (drill 0.4064) (layers "F.Cu" "B.Cu") (free) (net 1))
 (via (at 97.79 97.79) (size 0.8128) (drill 0.4064) (layers "F.Cu" "B.Cu") (free) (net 1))
 (via (at 87.63 105.41) (size 0.8128) (drill 0.4064) (layers "F.Cu" "B.Cu") (free) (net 1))
 (via (at 90.17 116.84) (size 0.8128) (drill 0.4064) (layers "F.Cu" "B.Cu") (free) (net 1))
 (via (at 101.6 91.44) (size 0.8128) (drill 0.4064) (layers "F.Cu" "B.Cu") (free) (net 1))
 (via (at 101.6 96.52) (size 0.8128) (drill 0.4064) (layers "F.Cu" "B.Cu") (free) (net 1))
 (via (at 87.63 97.79) (size 0.8128) (drill 0.4064) (layers "F.Cu" "B.Cu") (free) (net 1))
 (via (at 101.6 111.76) (size 0.8128) (drill 0.4064) (layers "F.Cu" "B.Cu") (free) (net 1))
 (via (at 95.25 99.06) (size 0.8128) (drill 0.4064) (layers "F.Cu" "B.Cu") (free) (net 1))
 (via (at 85.09 105.41) (size 0.8128) (drill 0.4064) (layers "F.Cu" "B.Cu") (free) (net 1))
 (via (at 99.06 86.36) (size 0.8128) (drill 0.4064) (layers "F.Cu" "B.Cu") (free) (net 1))
 (via (at 95.25 93.98) (size 0.8128) (drill 0.4064) (layers "F.Cu" "B.Cu") (free) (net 1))
 (segment (start 99.1 103.465) (end 99.1 101.6) (width 0.779374) (layer "F.Cu") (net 2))
 (segment (start 81.78 106.68) (end 95.885 106.68) (width 0.779374) (layer "F.Cu") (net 2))
 (segment (start 95.885 106.68) (end 99.1 103.465) (width 0.779374) (layer "F.Cu") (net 2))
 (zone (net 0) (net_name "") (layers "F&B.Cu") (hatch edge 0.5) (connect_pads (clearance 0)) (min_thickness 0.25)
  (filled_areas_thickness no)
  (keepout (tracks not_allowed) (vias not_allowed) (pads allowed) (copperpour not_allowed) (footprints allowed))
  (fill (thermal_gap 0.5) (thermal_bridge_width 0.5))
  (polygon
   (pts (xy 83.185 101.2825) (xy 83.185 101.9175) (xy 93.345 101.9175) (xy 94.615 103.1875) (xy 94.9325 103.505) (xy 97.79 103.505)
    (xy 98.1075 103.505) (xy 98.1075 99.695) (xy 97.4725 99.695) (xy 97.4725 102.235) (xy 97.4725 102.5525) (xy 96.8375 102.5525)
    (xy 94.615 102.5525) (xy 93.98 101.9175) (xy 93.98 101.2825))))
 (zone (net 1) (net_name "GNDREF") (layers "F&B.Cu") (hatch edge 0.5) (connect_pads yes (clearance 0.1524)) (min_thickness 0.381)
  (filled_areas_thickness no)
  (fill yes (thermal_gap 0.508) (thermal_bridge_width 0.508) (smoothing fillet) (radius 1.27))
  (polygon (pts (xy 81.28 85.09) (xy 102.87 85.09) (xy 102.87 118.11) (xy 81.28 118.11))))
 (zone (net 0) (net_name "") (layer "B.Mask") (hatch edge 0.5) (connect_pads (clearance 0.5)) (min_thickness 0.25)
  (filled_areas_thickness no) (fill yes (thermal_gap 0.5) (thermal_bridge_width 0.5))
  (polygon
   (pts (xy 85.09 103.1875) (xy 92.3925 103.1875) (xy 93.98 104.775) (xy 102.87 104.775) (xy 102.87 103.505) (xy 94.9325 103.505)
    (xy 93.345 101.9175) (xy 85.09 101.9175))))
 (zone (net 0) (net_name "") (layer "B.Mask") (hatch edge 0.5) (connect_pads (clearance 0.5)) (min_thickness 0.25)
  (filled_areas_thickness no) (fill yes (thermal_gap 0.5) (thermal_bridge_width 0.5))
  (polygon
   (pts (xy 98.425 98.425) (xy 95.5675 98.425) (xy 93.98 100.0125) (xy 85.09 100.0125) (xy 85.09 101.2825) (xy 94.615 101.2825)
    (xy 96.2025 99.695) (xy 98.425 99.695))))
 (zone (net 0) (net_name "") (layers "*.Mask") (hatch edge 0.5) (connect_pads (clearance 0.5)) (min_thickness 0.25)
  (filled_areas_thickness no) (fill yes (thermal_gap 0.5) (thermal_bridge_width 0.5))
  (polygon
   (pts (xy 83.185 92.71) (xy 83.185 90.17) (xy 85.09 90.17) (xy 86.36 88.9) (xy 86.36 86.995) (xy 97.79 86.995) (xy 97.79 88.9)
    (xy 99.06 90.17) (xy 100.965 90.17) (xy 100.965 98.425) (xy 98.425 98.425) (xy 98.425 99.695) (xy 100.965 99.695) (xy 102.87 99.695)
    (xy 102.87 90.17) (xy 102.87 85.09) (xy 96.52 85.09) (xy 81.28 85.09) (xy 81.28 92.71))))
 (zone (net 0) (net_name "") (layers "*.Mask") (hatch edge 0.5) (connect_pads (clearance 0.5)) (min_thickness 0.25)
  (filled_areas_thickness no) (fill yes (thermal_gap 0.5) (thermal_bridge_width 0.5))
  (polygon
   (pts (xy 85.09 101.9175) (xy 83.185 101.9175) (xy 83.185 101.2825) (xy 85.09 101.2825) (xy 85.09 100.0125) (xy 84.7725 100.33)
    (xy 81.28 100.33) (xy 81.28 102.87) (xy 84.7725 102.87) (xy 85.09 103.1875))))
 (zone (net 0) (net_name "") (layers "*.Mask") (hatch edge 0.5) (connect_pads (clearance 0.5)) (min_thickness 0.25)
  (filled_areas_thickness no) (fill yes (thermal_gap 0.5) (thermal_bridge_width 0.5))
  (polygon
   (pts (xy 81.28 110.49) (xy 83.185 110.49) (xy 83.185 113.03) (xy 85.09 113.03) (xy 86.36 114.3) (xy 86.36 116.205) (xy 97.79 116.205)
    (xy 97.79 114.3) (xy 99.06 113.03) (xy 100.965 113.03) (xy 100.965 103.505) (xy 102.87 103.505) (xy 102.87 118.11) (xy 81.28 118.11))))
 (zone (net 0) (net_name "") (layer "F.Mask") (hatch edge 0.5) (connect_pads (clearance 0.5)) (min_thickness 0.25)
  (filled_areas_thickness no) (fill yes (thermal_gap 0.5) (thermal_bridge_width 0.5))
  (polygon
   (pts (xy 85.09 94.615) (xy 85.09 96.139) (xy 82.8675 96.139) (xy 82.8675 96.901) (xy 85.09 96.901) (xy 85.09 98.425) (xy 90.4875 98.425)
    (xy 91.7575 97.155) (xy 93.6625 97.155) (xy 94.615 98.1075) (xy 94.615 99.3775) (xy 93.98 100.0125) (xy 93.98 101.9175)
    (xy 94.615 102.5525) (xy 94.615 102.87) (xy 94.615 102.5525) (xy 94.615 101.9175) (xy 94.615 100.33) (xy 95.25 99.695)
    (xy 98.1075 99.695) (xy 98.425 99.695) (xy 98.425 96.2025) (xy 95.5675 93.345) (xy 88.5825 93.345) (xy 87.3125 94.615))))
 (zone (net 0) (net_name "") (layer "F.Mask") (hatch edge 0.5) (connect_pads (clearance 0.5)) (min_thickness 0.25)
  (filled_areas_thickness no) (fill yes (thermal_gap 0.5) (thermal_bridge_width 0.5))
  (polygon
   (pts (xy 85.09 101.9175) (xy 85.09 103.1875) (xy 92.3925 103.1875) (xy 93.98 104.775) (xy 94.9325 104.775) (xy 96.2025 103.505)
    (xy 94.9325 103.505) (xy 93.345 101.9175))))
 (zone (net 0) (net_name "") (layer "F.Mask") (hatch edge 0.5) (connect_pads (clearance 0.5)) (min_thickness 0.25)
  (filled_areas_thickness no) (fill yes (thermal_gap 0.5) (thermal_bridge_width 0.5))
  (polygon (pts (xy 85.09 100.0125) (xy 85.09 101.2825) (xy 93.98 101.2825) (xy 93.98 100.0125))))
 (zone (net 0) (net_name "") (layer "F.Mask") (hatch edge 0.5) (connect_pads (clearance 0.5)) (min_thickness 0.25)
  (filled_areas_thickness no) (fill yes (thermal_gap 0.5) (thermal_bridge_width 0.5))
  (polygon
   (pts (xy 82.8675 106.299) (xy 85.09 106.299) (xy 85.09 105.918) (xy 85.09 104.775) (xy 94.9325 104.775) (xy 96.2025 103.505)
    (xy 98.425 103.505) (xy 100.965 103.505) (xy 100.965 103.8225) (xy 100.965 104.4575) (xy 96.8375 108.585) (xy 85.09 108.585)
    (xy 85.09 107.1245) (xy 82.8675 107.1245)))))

